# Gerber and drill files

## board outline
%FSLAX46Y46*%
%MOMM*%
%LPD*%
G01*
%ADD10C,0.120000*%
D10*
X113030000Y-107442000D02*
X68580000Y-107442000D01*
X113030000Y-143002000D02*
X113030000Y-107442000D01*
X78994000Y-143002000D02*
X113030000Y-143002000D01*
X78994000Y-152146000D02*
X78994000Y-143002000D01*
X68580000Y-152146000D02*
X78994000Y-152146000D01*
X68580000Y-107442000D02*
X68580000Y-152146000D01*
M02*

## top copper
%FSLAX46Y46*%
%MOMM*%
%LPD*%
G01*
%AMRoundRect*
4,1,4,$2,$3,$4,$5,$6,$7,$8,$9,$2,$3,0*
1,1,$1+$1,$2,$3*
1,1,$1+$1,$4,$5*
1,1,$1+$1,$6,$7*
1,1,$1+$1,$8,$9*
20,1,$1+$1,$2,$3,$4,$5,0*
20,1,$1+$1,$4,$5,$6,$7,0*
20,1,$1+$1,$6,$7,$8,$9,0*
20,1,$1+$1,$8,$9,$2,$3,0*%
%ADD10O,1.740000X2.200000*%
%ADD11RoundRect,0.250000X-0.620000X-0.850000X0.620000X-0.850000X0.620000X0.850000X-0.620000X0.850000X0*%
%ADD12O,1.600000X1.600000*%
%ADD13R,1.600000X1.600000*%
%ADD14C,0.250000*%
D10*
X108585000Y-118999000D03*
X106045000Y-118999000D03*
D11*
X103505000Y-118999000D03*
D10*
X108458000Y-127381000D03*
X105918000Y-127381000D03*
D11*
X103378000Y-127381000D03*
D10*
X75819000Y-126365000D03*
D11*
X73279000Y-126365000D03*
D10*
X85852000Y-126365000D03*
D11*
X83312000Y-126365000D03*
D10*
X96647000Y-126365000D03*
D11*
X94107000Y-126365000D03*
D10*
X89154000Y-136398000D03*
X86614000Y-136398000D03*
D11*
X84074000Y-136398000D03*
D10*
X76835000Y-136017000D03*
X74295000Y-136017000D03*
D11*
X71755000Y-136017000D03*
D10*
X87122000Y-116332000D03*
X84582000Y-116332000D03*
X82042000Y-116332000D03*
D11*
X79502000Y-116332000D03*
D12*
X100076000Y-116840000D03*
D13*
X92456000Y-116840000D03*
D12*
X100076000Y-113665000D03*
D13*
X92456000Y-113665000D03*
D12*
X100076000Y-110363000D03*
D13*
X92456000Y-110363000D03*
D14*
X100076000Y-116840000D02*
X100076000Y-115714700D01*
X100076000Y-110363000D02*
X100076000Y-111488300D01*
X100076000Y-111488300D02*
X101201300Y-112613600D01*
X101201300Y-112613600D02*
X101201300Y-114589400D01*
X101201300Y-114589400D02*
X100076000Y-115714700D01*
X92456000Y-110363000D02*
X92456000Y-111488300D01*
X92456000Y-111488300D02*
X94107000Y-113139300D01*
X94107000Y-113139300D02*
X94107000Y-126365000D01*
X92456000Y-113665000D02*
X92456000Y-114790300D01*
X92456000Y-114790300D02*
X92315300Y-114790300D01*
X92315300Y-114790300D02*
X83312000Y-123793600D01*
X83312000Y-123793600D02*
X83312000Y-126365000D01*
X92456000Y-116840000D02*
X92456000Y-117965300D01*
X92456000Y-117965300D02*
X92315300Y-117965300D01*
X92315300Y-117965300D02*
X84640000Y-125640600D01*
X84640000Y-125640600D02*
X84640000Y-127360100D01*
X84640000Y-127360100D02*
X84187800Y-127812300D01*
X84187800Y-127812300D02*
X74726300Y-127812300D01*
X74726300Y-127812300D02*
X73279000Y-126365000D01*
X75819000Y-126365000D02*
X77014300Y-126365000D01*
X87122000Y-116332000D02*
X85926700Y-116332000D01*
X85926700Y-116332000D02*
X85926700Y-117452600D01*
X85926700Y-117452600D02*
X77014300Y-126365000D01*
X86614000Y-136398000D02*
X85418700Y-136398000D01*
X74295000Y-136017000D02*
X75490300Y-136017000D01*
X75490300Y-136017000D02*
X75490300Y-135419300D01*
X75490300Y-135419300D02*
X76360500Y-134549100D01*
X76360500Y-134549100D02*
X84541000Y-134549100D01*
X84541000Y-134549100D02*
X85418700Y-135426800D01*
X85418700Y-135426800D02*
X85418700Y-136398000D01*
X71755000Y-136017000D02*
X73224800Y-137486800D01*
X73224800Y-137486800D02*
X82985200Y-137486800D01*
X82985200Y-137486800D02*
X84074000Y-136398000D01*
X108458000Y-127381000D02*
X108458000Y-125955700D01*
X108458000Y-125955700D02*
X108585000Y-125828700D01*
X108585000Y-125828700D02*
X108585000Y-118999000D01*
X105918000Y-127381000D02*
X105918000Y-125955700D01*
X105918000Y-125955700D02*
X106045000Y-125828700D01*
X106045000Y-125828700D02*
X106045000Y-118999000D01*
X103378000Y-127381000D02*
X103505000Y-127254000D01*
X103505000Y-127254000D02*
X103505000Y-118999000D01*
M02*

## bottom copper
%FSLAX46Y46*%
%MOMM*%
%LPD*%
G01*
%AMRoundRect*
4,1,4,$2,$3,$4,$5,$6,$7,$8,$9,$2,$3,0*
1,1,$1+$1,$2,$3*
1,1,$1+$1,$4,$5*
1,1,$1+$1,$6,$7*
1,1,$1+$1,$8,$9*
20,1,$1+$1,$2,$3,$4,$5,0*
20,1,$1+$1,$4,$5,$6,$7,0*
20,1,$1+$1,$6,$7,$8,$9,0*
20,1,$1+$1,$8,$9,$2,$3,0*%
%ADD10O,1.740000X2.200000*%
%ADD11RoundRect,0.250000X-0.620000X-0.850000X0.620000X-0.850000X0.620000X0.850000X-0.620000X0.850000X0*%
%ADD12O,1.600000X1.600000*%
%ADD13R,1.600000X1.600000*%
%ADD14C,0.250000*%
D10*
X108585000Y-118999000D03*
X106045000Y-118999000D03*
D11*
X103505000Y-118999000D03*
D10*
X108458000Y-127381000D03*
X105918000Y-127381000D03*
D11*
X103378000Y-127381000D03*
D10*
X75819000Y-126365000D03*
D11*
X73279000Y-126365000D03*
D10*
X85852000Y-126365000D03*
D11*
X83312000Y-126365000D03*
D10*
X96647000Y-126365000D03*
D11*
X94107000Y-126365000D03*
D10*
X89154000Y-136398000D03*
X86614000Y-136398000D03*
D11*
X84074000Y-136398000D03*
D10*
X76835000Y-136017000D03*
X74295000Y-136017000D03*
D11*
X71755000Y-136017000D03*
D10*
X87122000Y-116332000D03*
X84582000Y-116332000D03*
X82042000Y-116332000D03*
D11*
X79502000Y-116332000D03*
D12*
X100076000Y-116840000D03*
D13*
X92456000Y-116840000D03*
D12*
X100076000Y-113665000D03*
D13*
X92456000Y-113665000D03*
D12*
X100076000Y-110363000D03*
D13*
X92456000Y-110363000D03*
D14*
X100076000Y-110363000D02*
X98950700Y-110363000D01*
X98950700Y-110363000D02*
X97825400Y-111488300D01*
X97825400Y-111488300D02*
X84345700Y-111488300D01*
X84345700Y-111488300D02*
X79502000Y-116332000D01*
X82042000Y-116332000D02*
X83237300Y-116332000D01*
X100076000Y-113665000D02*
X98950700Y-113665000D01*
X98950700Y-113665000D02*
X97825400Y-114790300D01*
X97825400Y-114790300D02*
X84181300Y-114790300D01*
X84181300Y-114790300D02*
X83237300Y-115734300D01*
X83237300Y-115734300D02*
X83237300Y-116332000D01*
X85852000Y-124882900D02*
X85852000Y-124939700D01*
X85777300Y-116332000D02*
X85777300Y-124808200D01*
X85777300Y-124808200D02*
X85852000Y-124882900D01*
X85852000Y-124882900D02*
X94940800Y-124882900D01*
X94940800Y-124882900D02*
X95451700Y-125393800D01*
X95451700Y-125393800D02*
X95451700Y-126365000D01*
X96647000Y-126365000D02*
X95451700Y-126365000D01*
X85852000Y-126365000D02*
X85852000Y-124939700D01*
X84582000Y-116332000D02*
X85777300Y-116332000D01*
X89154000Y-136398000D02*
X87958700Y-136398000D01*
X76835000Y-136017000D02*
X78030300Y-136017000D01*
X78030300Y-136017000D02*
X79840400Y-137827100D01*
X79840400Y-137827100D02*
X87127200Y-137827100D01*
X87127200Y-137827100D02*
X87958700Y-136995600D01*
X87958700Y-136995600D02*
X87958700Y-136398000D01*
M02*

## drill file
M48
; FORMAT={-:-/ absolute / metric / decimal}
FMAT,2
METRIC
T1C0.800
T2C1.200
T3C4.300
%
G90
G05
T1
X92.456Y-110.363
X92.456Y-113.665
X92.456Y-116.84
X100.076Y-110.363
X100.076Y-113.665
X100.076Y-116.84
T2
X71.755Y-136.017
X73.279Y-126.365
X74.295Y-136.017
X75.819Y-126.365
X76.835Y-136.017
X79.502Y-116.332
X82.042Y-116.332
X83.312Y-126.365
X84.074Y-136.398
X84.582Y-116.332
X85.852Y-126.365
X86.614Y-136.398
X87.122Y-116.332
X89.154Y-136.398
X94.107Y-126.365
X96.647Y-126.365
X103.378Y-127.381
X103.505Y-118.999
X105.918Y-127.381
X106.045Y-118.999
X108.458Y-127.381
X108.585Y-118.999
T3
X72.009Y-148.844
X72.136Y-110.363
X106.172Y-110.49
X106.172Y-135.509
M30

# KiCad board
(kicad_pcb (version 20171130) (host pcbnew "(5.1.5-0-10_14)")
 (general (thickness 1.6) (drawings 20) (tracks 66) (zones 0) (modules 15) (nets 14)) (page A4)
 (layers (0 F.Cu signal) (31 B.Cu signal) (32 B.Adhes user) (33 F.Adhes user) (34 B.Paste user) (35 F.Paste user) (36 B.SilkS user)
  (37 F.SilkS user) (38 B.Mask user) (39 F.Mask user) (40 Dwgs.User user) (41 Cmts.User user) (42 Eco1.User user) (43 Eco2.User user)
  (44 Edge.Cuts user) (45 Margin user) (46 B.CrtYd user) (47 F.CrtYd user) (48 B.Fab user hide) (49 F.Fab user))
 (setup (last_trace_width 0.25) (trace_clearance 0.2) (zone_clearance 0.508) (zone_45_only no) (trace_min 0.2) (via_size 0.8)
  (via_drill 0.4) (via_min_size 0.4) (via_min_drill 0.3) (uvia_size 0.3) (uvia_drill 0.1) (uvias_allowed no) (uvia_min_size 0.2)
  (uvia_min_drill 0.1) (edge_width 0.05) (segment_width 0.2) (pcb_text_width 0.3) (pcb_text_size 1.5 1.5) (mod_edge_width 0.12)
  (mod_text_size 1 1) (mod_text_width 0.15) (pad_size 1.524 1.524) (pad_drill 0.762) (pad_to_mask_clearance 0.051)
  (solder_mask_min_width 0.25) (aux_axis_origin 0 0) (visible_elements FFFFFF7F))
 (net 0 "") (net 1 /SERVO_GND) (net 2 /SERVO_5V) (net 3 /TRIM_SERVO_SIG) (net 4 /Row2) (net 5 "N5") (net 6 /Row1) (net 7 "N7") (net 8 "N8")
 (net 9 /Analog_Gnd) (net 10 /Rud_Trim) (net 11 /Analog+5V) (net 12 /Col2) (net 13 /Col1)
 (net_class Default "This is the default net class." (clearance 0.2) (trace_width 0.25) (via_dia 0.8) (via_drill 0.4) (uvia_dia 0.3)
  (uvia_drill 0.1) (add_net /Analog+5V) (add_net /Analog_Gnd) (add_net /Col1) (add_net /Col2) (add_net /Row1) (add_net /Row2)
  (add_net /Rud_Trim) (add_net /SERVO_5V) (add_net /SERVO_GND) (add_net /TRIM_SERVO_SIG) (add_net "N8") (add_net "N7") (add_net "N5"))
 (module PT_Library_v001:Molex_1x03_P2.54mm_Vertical (layer F.Cu) (at 103.505 118.999)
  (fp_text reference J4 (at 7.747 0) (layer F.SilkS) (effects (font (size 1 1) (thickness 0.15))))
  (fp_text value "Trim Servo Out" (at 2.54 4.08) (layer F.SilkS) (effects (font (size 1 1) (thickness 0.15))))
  (pad 3 thru_hole oval (at 5.08 0) (size 1.74 2.2) (drill 1.2) (layers *.Cu *.Mask) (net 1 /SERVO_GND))
  (pad 2 thru_hole oval (at 2.54 0) (size 1.74 2.2) (drill 1.2) (layers *.Cu *.Mask) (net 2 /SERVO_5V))
  (pad 1 thru_hole roundrect (at 0 0) (size 1.74 2.2) (drill 1.2) (layers *.Cu *.Mask) (roundrect_rratio 0.143678) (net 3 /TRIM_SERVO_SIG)))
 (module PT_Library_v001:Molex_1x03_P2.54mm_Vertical (layer F.Cu) (at 103.378 127.381)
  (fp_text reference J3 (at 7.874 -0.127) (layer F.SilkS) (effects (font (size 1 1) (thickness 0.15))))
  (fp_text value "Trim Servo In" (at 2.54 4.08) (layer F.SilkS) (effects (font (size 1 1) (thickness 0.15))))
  (pad 3 thru_hole oval (at 5.08 0) (size 1.74 2.2) (drill 1.2) (layers *.Cu *.Mask) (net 1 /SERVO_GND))
  (pad 2 thru_hole oval (at 2.54 0) (size 1.74 2.2) (drill 1.2) (layers *.Cu *.Mask) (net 2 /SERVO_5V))
  (pad 1 thru_hole roundrect (at 0 0) (size 1.74 2.2) (drill 1.2) (layers *.Cu *.Mask) (roundrect_rratio 0.143678) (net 3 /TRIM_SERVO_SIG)))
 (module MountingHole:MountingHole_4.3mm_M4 (layer F.Cu) (at 72.009 148.844)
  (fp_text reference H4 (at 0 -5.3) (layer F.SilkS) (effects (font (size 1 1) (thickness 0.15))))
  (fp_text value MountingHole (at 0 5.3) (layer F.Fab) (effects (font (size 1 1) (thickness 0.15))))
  (pad 1 np_thru_hole circle (at 0 0) (size 4.3 4.3) (drill 4.3) (layers *.Cu *.Mask)))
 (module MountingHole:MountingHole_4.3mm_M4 (layer F.Cu) (at 106.172 135.509)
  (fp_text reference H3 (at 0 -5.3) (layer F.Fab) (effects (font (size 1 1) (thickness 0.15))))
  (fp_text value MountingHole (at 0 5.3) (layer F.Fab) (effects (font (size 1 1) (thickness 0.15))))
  (pad 1 np_thru_hole circle (at 0 0) (size 4.3 4.3) (drill 4.3) (layers *.Cu *.Mask)))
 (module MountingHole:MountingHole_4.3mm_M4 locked (layer F.Cu) (at 72.136 110.363)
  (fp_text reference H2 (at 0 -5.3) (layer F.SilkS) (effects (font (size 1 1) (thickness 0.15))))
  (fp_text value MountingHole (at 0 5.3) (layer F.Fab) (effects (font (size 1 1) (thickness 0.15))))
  (pad 1 np_thru_hole circle (at 0 0) (size 4.3 4.3) (drill 4.3) (layers *.Cu *.Mask)))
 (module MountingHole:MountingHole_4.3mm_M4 (layer F.Cu) (at 106.172 110.49)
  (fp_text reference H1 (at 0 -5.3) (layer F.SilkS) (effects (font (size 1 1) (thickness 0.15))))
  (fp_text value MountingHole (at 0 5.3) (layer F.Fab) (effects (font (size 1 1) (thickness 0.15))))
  (pad 1 np_thru_hole circle (at 0 0) (size 4.3 4.3) (drill 4.3) (layers *.Cu *.Mask)))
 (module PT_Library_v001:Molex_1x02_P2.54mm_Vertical (layer F.Cu) (at 73.279 126.365)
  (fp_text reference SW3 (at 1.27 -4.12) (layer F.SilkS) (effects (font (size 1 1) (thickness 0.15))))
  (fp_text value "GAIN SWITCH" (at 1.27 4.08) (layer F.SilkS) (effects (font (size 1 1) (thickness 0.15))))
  (pad 2 thru_hole oval (at 2.54 0) (size 1.74 2.2) (drill 1.2) (layers *.Cu *.Mask) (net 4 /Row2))
  (pad 1 thru_hole roundrect (at 0 0) (size 1.74 2.2) (drill 1.2) (layers *.Cu *.Mask) (roundrect_rratio 0.143678) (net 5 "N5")))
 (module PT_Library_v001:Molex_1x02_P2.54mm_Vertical (layer F.Cu) (at 83.312 126.365)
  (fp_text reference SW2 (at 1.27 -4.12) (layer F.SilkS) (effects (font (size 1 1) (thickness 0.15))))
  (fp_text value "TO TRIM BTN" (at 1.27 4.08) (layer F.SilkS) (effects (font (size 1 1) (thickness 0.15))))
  (pad 2 thru_hole oval (at 2.54 0) (size 1.74 2.2) (drill 1.2) (layers *.Cu *.Mask) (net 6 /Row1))
  (pad 1 thru_hole roundrect (at 0 0) (size 1.74 2.2) (drill 1.2) (layers *.Cu *.Mask) (roundrect_rratio 0.143678) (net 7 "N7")))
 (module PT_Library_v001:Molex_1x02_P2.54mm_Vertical (layer F.Cu) (at 94.107 126.365)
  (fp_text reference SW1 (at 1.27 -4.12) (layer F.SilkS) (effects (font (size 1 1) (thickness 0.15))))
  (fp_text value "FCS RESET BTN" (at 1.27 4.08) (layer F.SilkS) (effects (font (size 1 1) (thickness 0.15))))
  (pad 2 thru_hole oval (at 2.54 0) (size 1.74 2.2) (drill 1.2) (layers *.Cu *.Mask) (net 6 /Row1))
  (pad 1 thru_hole roundrect (at 0 0) (size 1.74 2.2) (drill 1.2) (layers *.Cu *.Mask) (roundrect_rratio 0.143678) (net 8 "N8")))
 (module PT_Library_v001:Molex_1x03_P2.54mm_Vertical (layer F.Cu) (at 84.074 136.398)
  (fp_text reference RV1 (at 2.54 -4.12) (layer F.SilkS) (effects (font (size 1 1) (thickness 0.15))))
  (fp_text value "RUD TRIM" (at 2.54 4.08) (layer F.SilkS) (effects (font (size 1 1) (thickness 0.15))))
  (pad 3 thru_hole oval (at 5.08 0) (size 1.74 2.2) (drill 1.2) (layers *.Cu *.Mask) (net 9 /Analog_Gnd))
  (pad 2 thru_hole oval (at 2.54 0) (size 1.74 2.2) (drill 1.2) (layers *.Cu *.Mask) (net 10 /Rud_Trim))
  (pad 1 thru_hole roundrect (at 0 0) (size 1.74 2.2) (drill 1.2) (layers *.Cu *.Mask) (roundrect_rratio 0.143678) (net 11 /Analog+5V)))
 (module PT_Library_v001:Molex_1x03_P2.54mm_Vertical (layer F.Cu) (at 71.755 136.017)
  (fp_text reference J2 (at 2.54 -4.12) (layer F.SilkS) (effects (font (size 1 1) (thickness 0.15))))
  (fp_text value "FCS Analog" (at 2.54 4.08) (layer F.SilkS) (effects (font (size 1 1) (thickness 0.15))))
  (pad 3 thru_hole oval (at 5.08 0) (size 1.74 2.2) (drill 1.2) (layers *.Cu *.Mask) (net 9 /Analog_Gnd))
  (pad 2 thru_hole oval (at 2.54 0) (size 1.74 2.2) (drill 1.2) (layers *.Cu *.Mask) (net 10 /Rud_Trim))
  (pad 1 thru_hole roundrect (at 0 0) (size 1.74 2.2) (drill 1.2) (layers *.Cu *.Mask) (roundrect_rratio 0.143678) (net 11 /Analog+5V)))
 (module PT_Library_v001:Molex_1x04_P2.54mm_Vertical (layer F.Cu) (at 79.502 116.332)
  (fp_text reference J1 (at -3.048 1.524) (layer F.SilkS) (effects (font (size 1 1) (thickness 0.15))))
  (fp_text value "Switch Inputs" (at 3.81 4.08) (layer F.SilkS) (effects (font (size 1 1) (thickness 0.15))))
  (pad 4 thru_hole oval (at 7.62 0) (size 1.74 2.2) (drill 1.2) (layers *.Cu *.Mask) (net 4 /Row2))
  (pad 3 thru_hole oval (at 5.08 0) (size 1.74 2.2) (drill 1.2) (layers *.Cu *.Mask) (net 6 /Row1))
  (pad 2 thru_hole oval (at 2.54 0) (size 1.74 2.2) (drill 1.2) (layers *.Cu *.Mask) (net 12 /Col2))
  (pad 1 thru_hole roundrect (at 0 0) (size 1.74 2.2) (drill 1.2) (layers *.Cu *.Mask) (roundrect_rratio 0.143678) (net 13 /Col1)))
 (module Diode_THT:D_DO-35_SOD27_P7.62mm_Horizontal (layer F.Cu) (at 92.456 116.84)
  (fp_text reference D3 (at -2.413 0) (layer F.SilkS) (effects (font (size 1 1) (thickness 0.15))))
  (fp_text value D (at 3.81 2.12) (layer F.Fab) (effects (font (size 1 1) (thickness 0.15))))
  (pad 2 thru_hole oval (at 7.62 0) (size 1.6 1.6) (drill 0.8) (layers *.Cu *.Mask) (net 13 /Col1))
  (pad 1 thru_hole rect (at 0 0) (size 1.6 1.6) (drill 0.8) (layers *.Cu *.Mask) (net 5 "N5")))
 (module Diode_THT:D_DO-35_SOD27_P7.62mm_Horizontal (layer F.Cu) (at 92.456 113.665)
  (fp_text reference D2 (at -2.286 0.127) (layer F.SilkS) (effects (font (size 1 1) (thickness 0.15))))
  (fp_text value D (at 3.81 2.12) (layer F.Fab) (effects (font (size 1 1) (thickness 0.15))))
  (pad 2 thru_hole oval (at 7.62 0) (size 1.6 1.6) (drill 0.8) (layers *.Cu *.Mask) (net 12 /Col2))
  (pad 1 thru_hole rect (at 0 0) (size 1.6 1.6) (drill 0.8) (layers *.Cu *.Mask) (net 7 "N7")))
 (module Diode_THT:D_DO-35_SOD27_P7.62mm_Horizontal (layer F.Cu) (at 92.456 110.363)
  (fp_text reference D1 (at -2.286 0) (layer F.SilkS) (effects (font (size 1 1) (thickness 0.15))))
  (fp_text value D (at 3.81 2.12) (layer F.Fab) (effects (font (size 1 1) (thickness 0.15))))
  (pad 2 thru_hole oval (at 7.62 0) (size 1.6 1.6) (drill 0.8) (layers *.Cu *.Mask) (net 13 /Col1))
  (pad 1 thru_hole rect (at 0 0) (size 1.6 1.6) (drill 0.8) (layers *.Cu *.Mask) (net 8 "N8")))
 (gr_line (start 113.03 107.442) (end 68.58 107.442) (layer Edge.Cuts) (width 0.12))
 (gr_line (start 113.03 143.002) (end 113.03 107.442) (layer Edge.Cuts) (width 0.12))
 (gr_line (start 78.994 143.002) (end 113.03 143.002) (layer Edge.Cuts) (width 0.12))
 (gr_line (start 78.994 152.146) (end 78.994 143.002) (layer Edge.Cuts) (width 0.12))
 (gr_line (start 68.58 152.146) (end 78.994 152.146) (layer Edge.Cuts) (width 0.12))
 (gr_line (start 68.58 107.442) (end 68.58 152.146) (layer Edge.Cuts) (width 0.12))
 (segment (start 100.076 116.84) (end 100.076 115.7147) (width 0.25) (layer F.Cu) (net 13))
 (segment (start 100.076 110.363) (end 100.076 111.4883) (width 0.25) (layer F.Cu) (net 13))
 (segment (start 100.076 111.4883) (end 101.2013 112.6136) (width 0.25) (layer F.Cu) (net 13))
 (segment (start 101.2013 112.6136) (end 101.2013 114.5894) (width 0.25) (layer F.Cu) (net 13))
 (segment (start 101.2013 114.5894) (end 100.076 115.7147) (width 0.25) (layer F.Cu) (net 13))
 (segment (start 100.076 110.363) (end 98.9507 110.363) (width 0.25) (layer B.Cu) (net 13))
 (segment (start 98.9507 110.363) (end 97.8254 111.4883) (width 0.25) (layer B.Cu) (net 13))
 (segment (start 97.8254 111.4883) (end 84.3457 111.4883) (width 0.25) (layer B.Cu) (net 13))
 (segment (start 84.3457 111.4883) (end 79.502 116.332) (width 0.25) (layer B.Cu) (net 13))
 (segment (start 92.456 110.363) (end 92.456 111.4883) (width 0.25) (layer F.Cu) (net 8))
 (segment (start 92.456 111.4883) (end 94.107 113.1393) (width 0.25) (layer F.Cu) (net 8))
 (segment (start 94.107 113.1393) (end 94.107 126.365) (width 0.25) (layer F.Cu) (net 8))
 (segment (start 82.042 116.332) (end 83.2373 116.332) (width 0.25) (layer B.Cu) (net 12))
 (segment (start 100.076 113.665) (end 98.9507 113.665) (width 0.25) (layer B.Cu) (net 12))
 (segment (start 98.9507 113.665) (end 97.8254 114.7903) (width 0.25) (layer B.Cu) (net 12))
 (segment (start 97.8254 114.7903) (end 84.1813 114.7903) (width 0.25) (layer B.Cu) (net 12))
 (segment (start 84.1813 114.7903) (end 83.2373 115.7343) (width 0.25) (layer B.Cu) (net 12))
 (segment (start 83.2373 115.7343) (end 83.2373 116.332) (width 0.25) (layer B.Cu) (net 12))
 (segment (start 92.456 113.665) (end 92.456 114.7903) (width 0.25) (layer F.Cu) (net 7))
 (segment (start 92.456 114.7903) (end 92.3153 114.7903) (width 0.25) (layer F.Cu) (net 7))
 (segment (start 92.3153 114.7903) (end 83.312 123.7936) (width 0.25) (layer F.Cu) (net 7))
 (segment (start 83.312 123.7936) (end 83.312 126.365) (width 0.25) (layer F.Cu) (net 7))
 (segment (start 92.456 116.84) (end 92.456 117.9653) (width 0.25) (layer F.Cu) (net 5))
 (segment (start 92.456 117.9653) (end 92.3153 117.9653) (width 0.25) (layer F.Cu) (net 5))
 (segment (start 92.3153 117.9653) (end 84.64 125.6406) (width 0.25) (layer F.Cu) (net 5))
 (segment (start 84.64 125.6406) (end 84.64 127.3601) (width 0.25) (layer F.Cu) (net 5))
 (segment (start 84.64 127.3601) (end 84.1878 127.8123) (width 0.25) (layer F.Cu) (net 5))
 (segment (start 84.1878 127.8123) (end 74.7263 127.8123) (width 0.25) (layer F.Cu) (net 5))
 (segment (start 74.7263 127.8123) (end 73.279 126.365) (width 0.25) (layer F.Cu) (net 5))
 (segment (start 75.819 126.365) (end 77.0143 126.365) (width 0.25) (layer F.Cu) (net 4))
 (segment (start 87.122 116.332) (end 85.9267 116.332) (width 0.25) (layer F.Cu) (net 4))
 (segment (start 85.9267 116.332) (end 85.9267 117.4526) (width 0.25) (layer F.Cu) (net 4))
 (segment (start 85.9267 117.4526) (end 77.0143 126.365) (width 0.25) (layer F.Cu) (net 4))
 (segment (start 85.852 124.8829) (end 85.852 124.9397) (width 0.25) (layer B.Cu) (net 6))
 (segment (start 85.7773 116.332) (end 85.7773 124.8082) (width 0.25) (layer B.Cu) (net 6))
 (segment (start 85.7773 124.8082) (end 85.852 124.8829) (width 0.25) (layer B.Cu) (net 6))
 (segment (start 85.852 124.8829) (end 94.9408 124.8829) (width 0.25) (layer B.Cu) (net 6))
 (segment (start 94.9408 124.8829) (end 95.4517 125.3938) (width 0.25) (layer B.Cu) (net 6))
 (segment (start 95.4517 125.3938) (end 95.4517 126.365) (width 0.25) (layer B.Cu) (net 6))
 (segment (start 96.647 126.365) (end 95.4517 126.365) (width 0.25) (layer B.Cu) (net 6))
 (segment (start 85.852 126.365) (end 85.852 124.9397) (width 0.25) (layer B.Cu) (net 6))
 (segment (start 84.582 116.332) (end 85.7773 116.332) (width 0.25) (layer B.Cu) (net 6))
 (segment (start 89.154 136.398) (end 87.9587 136.398) (width 0.25) (layer B.Cu) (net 9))
 (segment (start 76.835 136.017) (end 78.0303 136.017) (width 0.25) (layer B.Cu) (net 9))
 (segment (start 78.0303 136.017) (end 79.8404 137.8271) (width 0.25) (layer B.Cu) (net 9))
 (segment (start 79.8404 137.8271) (end 87.1272 137.8271) (width 0.25) (layer B.Cu) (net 9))
 (segment (start 87.1272 137.8271) (end 87.9587 136.9956) (width 0.25) (layer B.Cu) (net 9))
 (segment (start 87.9587 136.9956) (end 87.9587 136.398) (width 0.25) (layer B.Cu) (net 9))
 (segment (start 86.614 136.398) (end 85.4187 136.398) (width 0.25) (layer F.Cu) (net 10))
 (segment (start 74.295 136.017) (end 75.4903 136.017) (width 0.25) (layer F.Cu) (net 10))
 (segment (start 75.4903 136.017) (end 75.4903 135.4193) (width 0.25) (layer F.Cu) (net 10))
 (segment (start 75.4903 135.4193) (end 76.3605 134.5491) (width 0.25) (layer F.Cu) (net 10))
 (segment (start 76.3605 134.5491) (end 84.541 134.5491) (width 0.25) (layer F.Cu) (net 10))
 (segment (start 84.541 134.5491) (end 85.4187 135.4268) (width 0.25) (layer F.Cu) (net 10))
 (segment (start 85.4187 135.4268) (end 85.4187 136.398) (width 0.25) (layer F.Cu) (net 10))
 (segment (start 71.755 136.017) (end 73.2248 137.4868) (width 0.25) (layer F.Cu) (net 11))
 (segment (start 73.2248 137.4868) (end 82.9852 137.4868) (width 0.25) (layer F.Cu) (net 11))
 (segment (start 82.9852 137.4868) (end 84.074 136.398) (width 0.25) (layer F.Cu) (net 11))
 (segment (start 108.458 127.381) (end 108.458 125.9557) (width 0.25) (layer F.Cu) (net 1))
 (segment (start 108.458 125.9557) (end 108.585 125.8287) (width 0.25) (layer F.Cu) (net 1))
 (segment (start 108.585 125.8287) (end 108.585 118.999) (width 0.25) (layer F.Cu) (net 1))
 (segment (start 105.918 127.381) (end 105.918 125.9557) (width 0.25) (layer F.Cu) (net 2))
 (segment (start 105.918 125.9557) (end 106.045 125.8287) (width 0.25) (layer F.Cu) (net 2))
 (segment (start 106.045 125.8287) (end 106.045 118.999) (width 0.25) (layer F.Cu) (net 2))
 (segment (start 103.378 127.381) (end 103.505 127.254) (width 0.25) (layer F.Cu) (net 3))
 (segment (start 103.505 127.254) (end 103.505 118.999) (width 0.25) (layer F.Cu) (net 3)))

